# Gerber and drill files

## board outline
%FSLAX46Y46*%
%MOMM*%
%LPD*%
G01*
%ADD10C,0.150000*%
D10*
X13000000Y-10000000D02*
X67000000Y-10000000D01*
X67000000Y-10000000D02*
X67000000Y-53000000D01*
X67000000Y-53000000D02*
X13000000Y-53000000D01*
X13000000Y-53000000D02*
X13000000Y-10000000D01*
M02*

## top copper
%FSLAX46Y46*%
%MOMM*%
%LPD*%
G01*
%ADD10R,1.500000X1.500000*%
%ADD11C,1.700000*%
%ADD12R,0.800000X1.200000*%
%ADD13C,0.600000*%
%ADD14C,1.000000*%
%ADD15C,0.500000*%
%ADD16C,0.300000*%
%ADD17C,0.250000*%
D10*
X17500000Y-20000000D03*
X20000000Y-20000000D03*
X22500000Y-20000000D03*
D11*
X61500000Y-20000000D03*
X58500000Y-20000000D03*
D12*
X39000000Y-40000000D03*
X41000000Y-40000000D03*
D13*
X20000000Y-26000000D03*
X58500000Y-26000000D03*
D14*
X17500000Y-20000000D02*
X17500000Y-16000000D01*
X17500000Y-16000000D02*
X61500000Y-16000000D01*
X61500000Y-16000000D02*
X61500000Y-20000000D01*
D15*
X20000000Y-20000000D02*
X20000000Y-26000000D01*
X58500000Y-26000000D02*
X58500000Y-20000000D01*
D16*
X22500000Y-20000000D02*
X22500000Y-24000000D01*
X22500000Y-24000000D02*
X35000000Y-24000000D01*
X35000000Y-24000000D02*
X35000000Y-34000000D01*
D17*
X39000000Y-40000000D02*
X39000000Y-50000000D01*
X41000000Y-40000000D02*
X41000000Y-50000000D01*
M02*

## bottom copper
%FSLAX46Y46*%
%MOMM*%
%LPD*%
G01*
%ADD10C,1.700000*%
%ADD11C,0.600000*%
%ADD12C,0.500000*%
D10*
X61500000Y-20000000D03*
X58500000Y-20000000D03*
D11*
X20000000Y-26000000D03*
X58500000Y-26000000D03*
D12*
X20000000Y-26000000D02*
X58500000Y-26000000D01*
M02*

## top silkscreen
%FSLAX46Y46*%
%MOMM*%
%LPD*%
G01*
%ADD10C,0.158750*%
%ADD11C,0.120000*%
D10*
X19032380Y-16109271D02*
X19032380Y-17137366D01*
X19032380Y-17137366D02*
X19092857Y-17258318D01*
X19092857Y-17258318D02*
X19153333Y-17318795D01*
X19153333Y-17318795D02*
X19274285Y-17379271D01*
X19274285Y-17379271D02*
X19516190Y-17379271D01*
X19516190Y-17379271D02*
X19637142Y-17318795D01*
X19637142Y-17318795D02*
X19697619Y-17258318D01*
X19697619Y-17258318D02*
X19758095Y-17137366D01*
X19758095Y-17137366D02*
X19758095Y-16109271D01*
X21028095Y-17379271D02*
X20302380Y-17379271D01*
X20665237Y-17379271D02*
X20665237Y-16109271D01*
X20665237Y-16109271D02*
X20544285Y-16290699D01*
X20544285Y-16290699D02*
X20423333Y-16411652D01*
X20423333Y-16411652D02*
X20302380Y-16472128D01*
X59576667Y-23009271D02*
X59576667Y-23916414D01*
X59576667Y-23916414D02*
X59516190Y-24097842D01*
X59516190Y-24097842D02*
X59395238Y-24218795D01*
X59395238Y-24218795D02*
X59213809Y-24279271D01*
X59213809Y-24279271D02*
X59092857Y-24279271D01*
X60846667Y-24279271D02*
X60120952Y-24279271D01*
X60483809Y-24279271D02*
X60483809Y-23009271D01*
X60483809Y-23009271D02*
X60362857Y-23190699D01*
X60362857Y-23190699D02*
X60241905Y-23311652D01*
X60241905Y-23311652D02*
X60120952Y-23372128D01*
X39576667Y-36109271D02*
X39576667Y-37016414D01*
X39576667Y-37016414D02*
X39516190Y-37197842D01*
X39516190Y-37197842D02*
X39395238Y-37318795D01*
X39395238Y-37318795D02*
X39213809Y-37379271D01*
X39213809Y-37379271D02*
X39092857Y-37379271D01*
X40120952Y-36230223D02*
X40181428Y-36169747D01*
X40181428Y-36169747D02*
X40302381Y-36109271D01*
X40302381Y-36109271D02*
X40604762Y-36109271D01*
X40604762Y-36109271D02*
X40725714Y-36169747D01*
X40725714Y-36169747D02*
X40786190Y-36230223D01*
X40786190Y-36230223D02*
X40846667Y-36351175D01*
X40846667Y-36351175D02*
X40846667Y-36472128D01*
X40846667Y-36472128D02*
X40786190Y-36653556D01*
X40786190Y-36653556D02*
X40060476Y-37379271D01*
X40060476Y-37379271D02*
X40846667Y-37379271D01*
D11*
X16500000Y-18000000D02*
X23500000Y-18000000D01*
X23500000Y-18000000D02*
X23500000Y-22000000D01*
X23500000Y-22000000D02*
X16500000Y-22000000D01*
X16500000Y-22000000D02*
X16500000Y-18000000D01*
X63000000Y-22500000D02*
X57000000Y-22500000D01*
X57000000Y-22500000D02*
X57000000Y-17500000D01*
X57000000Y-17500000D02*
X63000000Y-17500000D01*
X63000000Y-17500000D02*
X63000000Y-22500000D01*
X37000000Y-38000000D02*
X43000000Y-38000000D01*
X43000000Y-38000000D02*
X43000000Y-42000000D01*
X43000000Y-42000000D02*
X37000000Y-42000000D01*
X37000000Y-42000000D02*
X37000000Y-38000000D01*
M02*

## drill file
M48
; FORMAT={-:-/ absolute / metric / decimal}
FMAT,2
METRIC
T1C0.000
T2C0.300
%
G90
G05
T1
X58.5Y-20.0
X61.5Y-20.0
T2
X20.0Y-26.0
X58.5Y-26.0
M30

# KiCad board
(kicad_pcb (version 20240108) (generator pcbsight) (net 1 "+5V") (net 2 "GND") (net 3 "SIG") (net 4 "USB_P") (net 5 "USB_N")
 (gr_line (start 13 10) (end 67 10) (layer "Edge.Cuts") (width 0.15))
 (gr_line (start 67 10) (end 67 53) (layer "Edge.Cuts") (width 0.15))
 (gr_line (start 67 53) (end 13 53) (layer "Edge.Cuts") (width 0.15))
 (gr_line (start 13 53) (end 13 10) (layer "Edge.Cuts") (width 0.15))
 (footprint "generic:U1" (at 20 20 0) (layer "F.Cu") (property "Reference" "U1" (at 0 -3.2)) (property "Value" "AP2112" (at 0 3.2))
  (fp_line (start -3.5 -2.0) (end 3.5 -2.0) (layer "F.SilkS") (width 0.12))
  (fp_line (start 3.5 -2.0) (end 3.5 2.0) (layer "F.SilkS") (width 0.12))
  (fp_line (start 3.5 2.0) (end -3.5 2.0) (layer "F.SilkS") (width 0.12))
  (fp_line (start -3.5 2.0) (end -3.5 -2.0) (layer "F.SilkS") (width 0.12))
  (pad "1" smd rect (at -2.5 0) (size 1.5 1.5) (layers "F.Cu" "F.Mask") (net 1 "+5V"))
  (pad "2" smd rect (at 0 0) (size 1.5 1.5) (layers "F.Cu" "F.Mask") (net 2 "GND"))
  (pad "3" smd rect (at 2.5 0) (size 1.5 1.5) (layers "F.Cu" "F.Mask") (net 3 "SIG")))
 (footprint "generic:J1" (at 60 20 180) (layer "F.Cu") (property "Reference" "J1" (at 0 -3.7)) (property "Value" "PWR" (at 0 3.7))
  (fp_line (start -3.0 -2.5) (end 3.0 -2.5) (layer "F.SilkS") (width 0.12))
  (fp_line (start 3.0 -2.5) (end 3.0 2.5) (layer "F.SilkS") (width 0.12))
  (fp_line (start 3.0 2.5) (end -3.0 2.5) (layer "F.SilkS") (width 0.12))
  (fp_line (start -3.0 2.5) (end -3.0 -2.5) (layer "F.SilkS") (width 0.12))
  (pad "1" thru_hole circle (at -1.5 0) (size 1.7 1.7) (layers "*.Cu" "*.Mask") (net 1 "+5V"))
  (pad "2" thru_hole circle (at 1.5 0) (size 1.7 1.7) (layers "*.Cu" "*.Mask") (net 2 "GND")))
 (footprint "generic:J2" (at 40 40 0) (layer "F.Cu") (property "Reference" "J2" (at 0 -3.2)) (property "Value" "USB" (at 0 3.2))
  (fp_line (start -3.0 -2.0) (end 3.0 -2.0) (layer "F.SilkS") (width 0.12))
  (fp_line (start 3.0 -2.0) (end 3.0 2.0) (layer "F.SilkS") (width 0.12))
  (fp_line (start 3.0 2.0) (end -3.0 2.0) (layer "F.SilkS") (width 0.12))
  (fp_line (start -3.0 2.0) (end -3.0 -2.0) (layer "F.SilkS") (width 0.12))
  (pad "1" smd rect (at -1.0 0) (size 0.8 1.2) (layers "F.Cu" "F.Mask") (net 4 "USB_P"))
  (pad "2" smd rect (at 1.0 0) (size 0.8 1.2) (layers "F.Cu" "F.Mask") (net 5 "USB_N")))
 (segment (start 17.5 20) (end 17.5 16) (width 1.0) (layer "F.Cu") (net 1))
 (segment (start 17.5 16) (end 61.5 16) (width 1.0) (layer "F.Cu") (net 1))
 (segment (start 61.5 16) (end 61.5 20) (width 1.0) (layer "F.Cu") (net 1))
 (segment (start 20 20) (end 20 26) (width 0.5) (layer "F.Cu") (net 2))
 (via (at 20 26) (size 0.6) (drill 0.3) (layers "F.Cu" "B.Cu") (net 2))
 (segment (start 20 26) (end 58.5 26) (width 0.5) (layer "B.Cu") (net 2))
 (via (at 58.5 26) (size 0.6) (drill 0.3) (layers "F.Cu" "B.Cu") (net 2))
 (segment (start 58.5 26) (end 58.5 20) (width 0.5) (layer "F.Cu") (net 2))
 (segment (start 22.5 20) (end 22.5 24) (width 0.3) (layer "F.Cu") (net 3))
 (segment (start 22.5 24) (end 35 24) (width 0.3) (layer "F.Cu") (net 3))
 (segment (start 35 24) (end 35 34) (width 0.3) (layer "F.Cu") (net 3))
 (segment (start 39 40) (end 39 50) (width 0.25) (layer "F.Cu") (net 4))
 (segment (start 41 40) (end 41 50) (width 0.25) (layer "F.Cu") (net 5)))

